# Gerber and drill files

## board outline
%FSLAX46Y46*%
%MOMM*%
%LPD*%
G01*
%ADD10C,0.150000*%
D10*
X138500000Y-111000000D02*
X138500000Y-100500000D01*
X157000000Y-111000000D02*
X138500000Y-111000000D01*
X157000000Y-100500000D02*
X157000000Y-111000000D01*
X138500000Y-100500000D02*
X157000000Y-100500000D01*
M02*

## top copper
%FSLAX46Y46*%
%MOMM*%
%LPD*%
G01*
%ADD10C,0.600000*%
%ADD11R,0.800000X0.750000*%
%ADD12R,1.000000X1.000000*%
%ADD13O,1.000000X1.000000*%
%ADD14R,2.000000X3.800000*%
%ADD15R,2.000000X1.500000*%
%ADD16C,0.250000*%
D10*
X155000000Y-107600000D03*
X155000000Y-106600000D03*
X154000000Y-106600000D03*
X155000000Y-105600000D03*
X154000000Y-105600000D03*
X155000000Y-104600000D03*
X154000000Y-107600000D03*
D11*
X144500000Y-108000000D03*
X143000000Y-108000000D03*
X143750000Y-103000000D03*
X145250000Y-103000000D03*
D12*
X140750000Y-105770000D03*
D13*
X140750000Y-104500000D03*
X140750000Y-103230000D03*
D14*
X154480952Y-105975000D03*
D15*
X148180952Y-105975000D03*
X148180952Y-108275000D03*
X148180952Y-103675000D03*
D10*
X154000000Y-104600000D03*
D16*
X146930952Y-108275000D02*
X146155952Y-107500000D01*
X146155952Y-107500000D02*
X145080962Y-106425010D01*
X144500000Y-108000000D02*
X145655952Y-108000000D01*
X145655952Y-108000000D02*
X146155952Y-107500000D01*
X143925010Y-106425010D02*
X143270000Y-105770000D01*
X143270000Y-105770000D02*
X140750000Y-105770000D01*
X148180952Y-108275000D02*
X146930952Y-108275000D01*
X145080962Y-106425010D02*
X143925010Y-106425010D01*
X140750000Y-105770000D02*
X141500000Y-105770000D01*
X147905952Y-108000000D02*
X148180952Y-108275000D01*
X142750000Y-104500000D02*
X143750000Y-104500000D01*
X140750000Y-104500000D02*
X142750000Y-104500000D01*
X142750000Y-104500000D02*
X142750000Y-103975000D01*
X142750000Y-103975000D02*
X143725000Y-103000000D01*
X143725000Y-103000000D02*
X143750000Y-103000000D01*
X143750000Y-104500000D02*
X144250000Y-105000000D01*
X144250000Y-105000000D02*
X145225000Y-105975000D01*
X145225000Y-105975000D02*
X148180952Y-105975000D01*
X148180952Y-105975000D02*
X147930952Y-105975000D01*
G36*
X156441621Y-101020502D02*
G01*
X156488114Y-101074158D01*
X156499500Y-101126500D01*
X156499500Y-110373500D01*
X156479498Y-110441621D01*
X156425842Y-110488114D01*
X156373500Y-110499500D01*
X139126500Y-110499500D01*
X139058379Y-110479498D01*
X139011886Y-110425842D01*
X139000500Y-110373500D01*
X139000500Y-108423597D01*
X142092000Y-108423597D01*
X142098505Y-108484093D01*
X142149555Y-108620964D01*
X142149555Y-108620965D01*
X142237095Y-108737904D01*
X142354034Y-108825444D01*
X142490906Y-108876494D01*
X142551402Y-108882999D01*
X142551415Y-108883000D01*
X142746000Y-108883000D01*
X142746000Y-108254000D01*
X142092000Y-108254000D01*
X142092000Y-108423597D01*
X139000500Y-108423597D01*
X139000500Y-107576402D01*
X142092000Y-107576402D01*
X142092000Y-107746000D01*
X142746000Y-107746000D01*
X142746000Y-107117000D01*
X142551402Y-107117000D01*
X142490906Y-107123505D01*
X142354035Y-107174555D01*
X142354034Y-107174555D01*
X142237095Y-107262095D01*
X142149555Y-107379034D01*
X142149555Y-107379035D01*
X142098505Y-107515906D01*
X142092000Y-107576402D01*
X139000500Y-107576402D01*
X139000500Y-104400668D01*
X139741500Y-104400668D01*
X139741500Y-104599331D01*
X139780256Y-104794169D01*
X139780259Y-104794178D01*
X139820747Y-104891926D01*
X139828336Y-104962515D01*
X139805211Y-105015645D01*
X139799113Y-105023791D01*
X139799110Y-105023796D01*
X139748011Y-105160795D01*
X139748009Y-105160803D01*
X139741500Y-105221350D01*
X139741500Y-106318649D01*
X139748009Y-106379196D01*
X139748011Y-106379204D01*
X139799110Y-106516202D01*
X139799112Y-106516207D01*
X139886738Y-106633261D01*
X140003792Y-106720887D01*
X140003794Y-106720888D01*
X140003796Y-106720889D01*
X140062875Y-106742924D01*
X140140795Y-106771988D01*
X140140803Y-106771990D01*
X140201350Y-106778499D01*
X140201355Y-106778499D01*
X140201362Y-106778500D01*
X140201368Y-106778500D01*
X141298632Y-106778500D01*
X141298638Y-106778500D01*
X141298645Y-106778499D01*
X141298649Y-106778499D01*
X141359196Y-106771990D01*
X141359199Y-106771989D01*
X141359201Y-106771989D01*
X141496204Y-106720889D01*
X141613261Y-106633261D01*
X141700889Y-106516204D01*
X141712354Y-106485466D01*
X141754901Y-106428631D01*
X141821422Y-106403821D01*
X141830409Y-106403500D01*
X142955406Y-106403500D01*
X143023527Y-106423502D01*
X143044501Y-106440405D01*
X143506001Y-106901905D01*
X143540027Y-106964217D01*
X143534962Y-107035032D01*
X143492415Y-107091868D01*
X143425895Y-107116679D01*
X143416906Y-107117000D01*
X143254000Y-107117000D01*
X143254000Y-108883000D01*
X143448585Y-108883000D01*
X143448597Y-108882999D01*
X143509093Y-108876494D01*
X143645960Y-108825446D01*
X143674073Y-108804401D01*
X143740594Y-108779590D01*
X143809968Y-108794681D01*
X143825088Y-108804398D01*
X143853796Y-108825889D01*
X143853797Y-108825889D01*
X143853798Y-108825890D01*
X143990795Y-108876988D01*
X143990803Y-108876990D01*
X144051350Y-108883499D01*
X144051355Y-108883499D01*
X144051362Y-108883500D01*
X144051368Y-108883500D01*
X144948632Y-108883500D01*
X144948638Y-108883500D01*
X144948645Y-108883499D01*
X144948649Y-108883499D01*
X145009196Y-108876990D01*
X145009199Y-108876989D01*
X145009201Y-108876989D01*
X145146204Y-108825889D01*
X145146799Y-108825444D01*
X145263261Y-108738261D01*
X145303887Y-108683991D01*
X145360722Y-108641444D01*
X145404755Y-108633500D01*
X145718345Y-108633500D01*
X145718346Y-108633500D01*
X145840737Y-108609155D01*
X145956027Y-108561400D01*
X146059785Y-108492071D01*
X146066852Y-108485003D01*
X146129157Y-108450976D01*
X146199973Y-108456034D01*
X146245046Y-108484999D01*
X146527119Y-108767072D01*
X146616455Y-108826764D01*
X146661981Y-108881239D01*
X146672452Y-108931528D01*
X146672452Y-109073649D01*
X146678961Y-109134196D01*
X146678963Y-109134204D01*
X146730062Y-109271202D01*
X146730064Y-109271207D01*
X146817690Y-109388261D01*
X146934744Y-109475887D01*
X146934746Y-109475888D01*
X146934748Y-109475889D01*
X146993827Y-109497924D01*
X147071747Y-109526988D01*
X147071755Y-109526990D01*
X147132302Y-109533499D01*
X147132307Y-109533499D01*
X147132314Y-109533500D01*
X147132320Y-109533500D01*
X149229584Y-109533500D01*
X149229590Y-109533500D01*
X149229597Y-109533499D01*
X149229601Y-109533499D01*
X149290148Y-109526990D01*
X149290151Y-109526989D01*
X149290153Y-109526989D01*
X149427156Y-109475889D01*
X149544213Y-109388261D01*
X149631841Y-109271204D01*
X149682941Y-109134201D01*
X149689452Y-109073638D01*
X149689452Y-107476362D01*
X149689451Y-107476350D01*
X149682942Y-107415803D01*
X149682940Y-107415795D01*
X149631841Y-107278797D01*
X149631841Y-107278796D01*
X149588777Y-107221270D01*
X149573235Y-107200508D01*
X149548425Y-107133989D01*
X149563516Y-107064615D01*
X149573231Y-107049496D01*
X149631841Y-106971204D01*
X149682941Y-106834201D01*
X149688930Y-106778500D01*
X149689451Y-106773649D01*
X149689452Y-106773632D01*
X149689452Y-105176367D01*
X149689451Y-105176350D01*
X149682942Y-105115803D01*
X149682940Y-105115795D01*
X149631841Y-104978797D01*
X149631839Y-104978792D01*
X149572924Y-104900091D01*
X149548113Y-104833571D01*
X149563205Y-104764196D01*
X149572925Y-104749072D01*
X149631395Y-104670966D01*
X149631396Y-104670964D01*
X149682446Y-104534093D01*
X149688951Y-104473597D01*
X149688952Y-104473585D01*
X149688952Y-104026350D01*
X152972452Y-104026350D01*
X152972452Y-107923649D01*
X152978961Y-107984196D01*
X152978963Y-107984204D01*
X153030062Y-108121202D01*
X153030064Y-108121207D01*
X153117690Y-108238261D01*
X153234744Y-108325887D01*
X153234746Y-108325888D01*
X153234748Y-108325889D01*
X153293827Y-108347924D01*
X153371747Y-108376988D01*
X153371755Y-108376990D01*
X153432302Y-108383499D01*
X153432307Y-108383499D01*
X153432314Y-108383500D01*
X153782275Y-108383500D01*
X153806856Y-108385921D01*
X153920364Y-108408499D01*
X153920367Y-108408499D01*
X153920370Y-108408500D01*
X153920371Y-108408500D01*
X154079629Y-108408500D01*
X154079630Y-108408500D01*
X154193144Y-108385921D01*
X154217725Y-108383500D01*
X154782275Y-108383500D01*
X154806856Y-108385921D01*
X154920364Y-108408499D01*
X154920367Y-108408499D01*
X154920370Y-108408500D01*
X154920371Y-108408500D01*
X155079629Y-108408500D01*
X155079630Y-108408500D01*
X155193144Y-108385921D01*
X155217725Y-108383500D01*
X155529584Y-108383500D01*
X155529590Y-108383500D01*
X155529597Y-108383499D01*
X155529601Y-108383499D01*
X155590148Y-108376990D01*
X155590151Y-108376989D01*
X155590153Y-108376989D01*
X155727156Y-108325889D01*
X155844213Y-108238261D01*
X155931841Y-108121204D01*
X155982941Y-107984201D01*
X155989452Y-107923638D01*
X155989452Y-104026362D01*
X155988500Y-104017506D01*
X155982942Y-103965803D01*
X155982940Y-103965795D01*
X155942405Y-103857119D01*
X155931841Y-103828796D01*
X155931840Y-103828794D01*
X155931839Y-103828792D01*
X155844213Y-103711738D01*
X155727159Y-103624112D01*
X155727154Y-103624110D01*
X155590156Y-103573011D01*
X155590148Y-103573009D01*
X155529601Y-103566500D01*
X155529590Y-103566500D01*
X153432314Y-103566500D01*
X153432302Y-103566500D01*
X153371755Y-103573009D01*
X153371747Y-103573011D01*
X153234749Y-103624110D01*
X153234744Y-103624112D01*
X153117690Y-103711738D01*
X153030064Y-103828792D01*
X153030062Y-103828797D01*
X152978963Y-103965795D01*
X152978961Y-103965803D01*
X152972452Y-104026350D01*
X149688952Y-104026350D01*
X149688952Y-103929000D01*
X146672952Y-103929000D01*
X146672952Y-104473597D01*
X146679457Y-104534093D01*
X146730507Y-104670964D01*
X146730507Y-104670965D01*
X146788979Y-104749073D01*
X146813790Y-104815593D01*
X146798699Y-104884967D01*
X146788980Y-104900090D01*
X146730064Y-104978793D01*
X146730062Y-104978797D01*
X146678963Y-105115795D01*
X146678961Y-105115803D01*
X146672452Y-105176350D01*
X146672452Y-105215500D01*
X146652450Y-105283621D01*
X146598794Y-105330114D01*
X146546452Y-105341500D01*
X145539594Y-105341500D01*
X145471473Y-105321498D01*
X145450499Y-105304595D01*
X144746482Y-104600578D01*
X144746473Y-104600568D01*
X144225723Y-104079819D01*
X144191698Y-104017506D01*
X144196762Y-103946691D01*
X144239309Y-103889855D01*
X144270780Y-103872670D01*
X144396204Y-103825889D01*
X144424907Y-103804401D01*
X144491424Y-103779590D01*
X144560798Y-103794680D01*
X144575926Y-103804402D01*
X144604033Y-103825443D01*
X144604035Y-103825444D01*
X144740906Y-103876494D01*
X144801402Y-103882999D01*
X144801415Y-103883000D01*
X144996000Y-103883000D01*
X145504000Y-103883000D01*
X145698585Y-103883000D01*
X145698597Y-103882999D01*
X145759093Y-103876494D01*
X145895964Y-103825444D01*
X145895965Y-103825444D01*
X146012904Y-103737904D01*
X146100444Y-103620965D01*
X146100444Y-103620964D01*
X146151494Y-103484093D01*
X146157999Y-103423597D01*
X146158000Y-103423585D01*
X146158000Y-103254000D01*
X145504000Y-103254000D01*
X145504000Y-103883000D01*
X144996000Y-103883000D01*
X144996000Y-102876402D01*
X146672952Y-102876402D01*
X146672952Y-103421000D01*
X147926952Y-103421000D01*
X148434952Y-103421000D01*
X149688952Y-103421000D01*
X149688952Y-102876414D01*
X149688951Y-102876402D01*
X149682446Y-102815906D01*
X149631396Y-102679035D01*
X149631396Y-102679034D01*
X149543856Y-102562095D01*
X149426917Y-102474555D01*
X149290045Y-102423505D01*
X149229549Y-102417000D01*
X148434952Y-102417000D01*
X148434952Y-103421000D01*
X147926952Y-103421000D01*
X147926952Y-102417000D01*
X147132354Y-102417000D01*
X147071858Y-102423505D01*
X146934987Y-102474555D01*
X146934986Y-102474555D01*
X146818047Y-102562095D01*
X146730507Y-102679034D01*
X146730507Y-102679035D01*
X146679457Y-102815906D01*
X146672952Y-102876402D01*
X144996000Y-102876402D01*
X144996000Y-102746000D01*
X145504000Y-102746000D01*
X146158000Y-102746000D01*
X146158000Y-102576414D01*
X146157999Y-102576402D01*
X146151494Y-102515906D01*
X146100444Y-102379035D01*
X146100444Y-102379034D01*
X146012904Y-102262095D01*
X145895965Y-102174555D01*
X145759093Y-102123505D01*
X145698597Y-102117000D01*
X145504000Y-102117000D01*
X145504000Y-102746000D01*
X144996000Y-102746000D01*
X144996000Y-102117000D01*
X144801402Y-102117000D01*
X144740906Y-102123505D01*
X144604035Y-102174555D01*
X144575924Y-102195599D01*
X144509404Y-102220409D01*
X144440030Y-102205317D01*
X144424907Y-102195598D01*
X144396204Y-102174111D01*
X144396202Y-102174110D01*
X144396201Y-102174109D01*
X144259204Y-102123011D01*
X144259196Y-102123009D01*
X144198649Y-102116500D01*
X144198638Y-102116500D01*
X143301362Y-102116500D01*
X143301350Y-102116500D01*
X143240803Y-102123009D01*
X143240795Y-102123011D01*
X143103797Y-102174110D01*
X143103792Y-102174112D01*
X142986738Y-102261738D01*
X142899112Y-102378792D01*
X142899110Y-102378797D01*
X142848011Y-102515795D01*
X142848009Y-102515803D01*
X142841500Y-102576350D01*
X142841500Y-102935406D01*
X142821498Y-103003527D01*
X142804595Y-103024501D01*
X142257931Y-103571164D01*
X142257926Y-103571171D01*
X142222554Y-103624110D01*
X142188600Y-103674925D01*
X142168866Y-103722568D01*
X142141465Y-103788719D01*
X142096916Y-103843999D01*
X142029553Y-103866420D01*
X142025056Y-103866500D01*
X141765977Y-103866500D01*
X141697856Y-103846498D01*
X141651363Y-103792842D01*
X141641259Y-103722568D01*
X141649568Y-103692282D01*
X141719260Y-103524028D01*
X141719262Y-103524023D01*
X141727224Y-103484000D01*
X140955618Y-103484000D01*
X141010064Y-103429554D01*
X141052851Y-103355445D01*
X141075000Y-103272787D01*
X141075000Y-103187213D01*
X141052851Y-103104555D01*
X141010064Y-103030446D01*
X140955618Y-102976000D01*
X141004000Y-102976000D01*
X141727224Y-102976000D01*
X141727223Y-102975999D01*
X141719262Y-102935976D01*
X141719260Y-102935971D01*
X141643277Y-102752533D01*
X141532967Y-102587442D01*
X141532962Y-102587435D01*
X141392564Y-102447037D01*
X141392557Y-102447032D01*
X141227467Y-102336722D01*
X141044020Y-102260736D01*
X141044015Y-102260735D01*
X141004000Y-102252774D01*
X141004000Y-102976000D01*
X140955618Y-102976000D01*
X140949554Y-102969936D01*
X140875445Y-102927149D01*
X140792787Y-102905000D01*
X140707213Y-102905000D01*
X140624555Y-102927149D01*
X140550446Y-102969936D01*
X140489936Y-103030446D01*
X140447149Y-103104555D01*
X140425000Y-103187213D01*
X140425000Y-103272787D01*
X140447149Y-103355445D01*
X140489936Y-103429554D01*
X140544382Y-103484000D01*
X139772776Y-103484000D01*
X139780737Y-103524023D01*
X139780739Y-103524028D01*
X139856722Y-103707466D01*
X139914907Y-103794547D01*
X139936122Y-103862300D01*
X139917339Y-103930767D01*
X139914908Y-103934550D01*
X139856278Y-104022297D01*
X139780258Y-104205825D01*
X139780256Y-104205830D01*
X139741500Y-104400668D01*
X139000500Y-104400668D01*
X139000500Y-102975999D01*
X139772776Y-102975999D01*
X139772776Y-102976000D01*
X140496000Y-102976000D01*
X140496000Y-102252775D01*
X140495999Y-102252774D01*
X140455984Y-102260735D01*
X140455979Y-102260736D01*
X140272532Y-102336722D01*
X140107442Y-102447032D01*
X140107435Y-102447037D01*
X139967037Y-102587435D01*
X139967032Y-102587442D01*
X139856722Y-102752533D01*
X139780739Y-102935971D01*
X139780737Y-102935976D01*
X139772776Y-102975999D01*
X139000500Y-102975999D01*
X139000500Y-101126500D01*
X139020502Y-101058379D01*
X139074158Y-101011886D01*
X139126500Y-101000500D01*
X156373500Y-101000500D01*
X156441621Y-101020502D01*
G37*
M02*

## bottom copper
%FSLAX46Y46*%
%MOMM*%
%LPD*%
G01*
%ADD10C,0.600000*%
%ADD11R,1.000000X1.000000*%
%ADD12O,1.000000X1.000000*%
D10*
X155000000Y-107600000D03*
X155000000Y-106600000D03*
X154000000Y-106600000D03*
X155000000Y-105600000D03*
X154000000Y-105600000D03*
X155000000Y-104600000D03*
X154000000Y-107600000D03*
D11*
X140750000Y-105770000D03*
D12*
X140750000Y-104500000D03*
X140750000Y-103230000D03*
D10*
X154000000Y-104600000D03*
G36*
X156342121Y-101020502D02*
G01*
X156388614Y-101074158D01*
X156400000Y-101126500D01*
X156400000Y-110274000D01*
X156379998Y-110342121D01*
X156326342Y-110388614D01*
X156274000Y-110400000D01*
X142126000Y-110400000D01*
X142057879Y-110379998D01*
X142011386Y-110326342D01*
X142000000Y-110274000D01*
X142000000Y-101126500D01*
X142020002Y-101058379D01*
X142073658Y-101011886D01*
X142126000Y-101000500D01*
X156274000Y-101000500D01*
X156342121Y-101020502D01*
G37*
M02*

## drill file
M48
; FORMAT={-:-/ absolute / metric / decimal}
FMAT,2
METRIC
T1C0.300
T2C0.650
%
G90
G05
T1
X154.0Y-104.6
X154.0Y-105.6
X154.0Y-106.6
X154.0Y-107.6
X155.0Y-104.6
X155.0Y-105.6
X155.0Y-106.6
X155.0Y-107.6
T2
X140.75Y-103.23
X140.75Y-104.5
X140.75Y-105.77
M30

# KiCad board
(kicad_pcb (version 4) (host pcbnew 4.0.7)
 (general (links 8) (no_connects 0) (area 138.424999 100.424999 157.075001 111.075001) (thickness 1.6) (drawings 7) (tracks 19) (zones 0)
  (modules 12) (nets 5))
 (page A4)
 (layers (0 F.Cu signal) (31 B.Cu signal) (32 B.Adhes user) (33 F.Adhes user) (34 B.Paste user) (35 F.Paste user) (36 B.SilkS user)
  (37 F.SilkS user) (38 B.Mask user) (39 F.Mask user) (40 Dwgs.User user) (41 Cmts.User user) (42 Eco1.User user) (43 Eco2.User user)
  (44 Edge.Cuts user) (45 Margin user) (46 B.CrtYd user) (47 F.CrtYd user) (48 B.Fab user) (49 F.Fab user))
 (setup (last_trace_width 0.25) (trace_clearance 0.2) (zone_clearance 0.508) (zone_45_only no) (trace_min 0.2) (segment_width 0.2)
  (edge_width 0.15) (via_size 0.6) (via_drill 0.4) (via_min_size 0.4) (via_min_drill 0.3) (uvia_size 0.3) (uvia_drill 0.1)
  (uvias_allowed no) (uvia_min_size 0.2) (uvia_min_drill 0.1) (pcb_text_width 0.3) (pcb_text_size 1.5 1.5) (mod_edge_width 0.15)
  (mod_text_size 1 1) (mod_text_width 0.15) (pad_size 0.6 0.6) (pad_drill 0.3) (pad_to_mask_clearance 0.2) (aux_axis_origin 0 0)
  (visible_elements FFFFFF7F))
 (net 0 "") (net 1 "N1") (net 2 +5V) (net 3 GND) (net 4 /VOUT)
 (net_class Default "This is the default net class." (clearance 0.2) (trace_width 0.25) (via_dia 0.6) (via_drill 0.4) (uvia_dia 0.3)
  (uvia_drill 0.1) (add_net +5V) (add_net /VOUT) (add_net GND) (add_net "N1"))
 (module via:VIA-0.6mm (layer F.Cu) (at 155 107.6)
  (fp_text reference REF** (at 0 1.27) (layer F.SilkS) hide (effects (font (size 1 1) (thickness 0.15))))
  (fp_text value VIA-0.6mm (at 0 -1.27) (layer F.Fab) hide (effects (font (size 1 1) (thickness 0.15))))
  (pad 1 thru_hole circle (at 0 0) (size 0.6 0.6) (drill 0.3) (layers *.Cu) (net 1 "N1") (zone_connect 2)))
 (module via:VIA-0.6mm (layer F.Cu) (at 155 106.6)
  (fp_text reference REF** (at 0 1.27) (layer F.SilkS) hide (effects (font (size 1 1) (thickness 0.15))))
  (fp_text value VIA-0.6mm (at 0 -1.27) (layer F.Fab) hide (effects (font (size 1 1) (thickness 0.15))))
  (pad 1 thru_hole circle (at 0 0) (size 0.6 0.6) (drill 0.3) (layers *.Cu) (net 1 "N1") (zone_connect 2)))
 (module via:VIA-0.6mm (layer F.Cu) (at 154 106.6)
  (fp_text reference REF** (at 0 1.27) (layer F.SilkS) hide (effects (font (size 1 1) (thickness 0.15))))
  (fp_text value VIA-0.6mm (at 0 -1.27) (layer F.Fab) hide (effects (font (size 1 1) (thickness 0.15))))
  (pad 1 thru_hole circle (at 0 0) (size 0.6 0.6) (drill 0.3) (layers *.Cu) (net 1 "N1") (zone_connect 2)))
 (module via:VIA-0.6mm (layer F.Cu) (at 155 105.6)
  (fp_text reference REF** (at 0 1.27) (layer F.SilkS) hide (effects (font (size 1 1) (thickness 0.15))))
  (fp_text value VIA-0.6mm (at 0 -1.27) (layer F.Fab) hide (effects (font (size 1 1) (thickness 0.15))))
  (pad 1 thru_hole circle (at 0 0) (size 0.6 0.6) (drill 0.3) (layers *.Cu) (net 1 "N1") (zone_connect 2)))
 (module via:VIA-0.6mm (layer F.Cu) (at 154 105.6)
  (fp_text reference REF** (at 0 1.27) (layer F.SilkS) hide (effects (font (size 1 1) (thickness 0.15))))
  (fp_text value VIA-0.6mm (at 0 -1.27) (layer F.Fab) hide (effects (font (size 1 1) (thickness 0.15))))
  (pad 1 thru_hole circle (at 0 0) (size 0.6 0.6) (drill 0.3) (layers *.Cu) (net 1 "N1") (zone_connect 2)))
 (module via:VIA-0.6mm (layer F.Cu) (at 155 104.6)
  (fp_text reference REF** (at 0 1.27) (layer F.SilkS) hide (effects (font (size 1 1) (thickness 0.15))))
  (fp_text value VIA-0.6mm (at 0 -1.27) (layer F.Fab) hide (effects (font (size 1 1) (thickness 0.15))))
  (pad 1 thru_hole circle (at 0 0) (size 0.6 0.6) (drill 0.3) (layers *.Cu) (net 1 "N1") (zone_connect 2)))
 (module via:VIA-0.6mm (layer F.Cu) (at 154 107.6)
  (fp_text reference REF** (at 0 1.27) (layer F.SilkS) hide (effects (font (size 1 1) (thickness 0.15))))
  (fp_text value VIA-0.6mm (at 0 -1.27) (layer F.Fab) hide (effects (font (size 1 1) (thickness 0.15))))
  (pad 1 thru_hole circle (at 0 0) (size 0.6 0.6) (drill 0.3) (layers *.Cu) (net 1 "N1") (zone_connect 2)))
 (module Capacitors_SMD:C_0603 (layer F.Cu) (at 143.75 108 180)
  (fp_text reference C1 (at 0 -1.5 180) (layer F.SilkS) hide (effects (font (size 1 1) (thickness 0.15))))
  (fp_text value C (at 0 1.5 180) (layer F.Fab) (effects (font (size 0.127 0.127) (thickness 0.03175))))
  (pad 1 smd rect (at -0.75 0 180) (size 0.8 0.75) (layers F.Cu F.Paste F.Mask) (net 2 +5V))
  (pad 2 smd rect (at 0.75 0 180) (size 0.8 0.75) (layers F.Cu F.Paste F.Mask) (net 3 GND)))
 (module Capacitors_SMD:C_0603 (layer F.Cu) (at 144.5 103)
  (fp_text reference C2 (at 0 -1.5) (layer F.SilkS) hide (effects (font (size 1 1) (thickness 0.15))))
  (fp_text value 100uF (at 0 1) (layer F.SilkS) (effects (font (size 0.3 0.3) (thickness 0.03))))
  (pad 1 smd rect (at -0.75 0) (size 0.8 0.75) (layers F.Cu F.Paste F.Mask) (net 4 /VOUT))
  (pad 2 smd rect (at 0.75 0) (size 0.8 0.75) (layers F.Cu F.Paste F.Mask) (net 3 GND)))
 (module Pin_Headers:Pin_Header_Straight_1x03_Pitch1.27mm (layer F.Cu) (at 140.75 105.77 180)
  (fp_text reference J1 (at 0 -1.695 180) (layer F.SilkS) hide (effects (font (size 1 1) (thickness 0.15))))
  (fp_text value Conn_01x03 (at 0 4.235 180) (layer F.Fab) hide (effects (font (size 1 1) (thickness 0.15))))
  (pad 1 thru_hole rect (at 0 0 180) (size 1 1) (drill 0.65) (layers *.Cu *.Mask) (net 2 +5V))
  (pad 2 thru_hole oval (at 0 1.27 180) (size 1 1) (drill 0.65) (layers *.Cu *.Mask) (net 4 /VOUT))
  (pad 3 thru_hole oval (at 0 2.54 180) (size 1 1) (drill 0.65) (layers *.Cu *.Mask) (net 3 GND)))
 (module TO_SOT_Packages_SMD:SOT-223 (layer F.Cu) (at 151.330952 105.975)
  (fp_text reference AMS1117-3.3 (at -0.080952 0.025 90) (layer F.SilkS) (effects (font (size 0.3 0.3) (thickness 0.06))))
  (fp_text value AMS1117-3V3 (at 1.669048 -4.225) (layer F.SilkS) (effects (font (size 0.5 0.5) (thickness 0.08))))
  (pad 4 smd rect (at 3.15 0) (size 2 3.8) (layers F.Cu F.Paste F.Mask) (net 1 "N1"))
  (pad 2 smd rect (at -3.15 0) (size 2 1.5) (layers F.Cu F.Paste F.Mask) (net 4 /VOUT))
  (pad 3 smd rect (at -3.15 2.3) (size 2 1.5) (layers F.Cu F.Paste F.Mask) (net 2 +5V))
  (pad 1 smd rect (at -3.15 -2.3) (size 2 1.5) (layers F.Cu F.Paste F.Mask) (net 3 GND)))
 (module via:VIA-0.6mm (layer F.Cu) (at 154 104.6)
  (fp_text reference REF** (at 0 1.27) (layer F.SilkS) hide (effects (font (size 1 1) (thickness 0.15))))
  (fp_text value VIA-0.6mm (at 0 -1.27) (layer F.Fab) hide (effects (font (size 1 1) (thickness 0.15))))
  (pad 1 thru_hole circle (at 0 0) (size 0.6 0.6) (drill 0.3) (layers *.Cu) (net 1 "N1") (zone_connect 2)))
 (gr_line (start 138.5 111) (end 138.5 100.5) (angle 90) (layer Edge.Cuts) (width 0.15))
 (gr_line (start 157 111) (end 138.5 111) (angle 90) (layer Edge.Cuts) (width 0.15))
 (gr_line (start 157 100.5) (end 157 111) (angle 90) (layer Edge.Cuts) (width 0.15))
 (gr_line (start 138.5 100.5) (end 157 100.5) (angle 90) (layer Edge.Cuts) (width 0.15))
 (segment (start 146.930952 108.275) (end 146.155952 107.5) (width 0.25) (layer F.Cu) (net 2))
 (segment (start 146.155952 107.5) (end 145.080962 106.42501) (width 0.25) (layer F.Cu) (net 2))
 (segment (start 144.5 108) (end 145.655952 108) (width 0.25) (layer F.Cu) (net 2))
 (segment (start 145.655952 108) (end 146.155952 107.5) (width 0.25) (layer F.Cu) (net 2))
 (segment (start 143.92501 106.42501) (end 143.27 105.77) (width 0.25) (layer F.Cu) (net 2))
 (segment (start 143.27 105.77) (end 140.75 105.77) (width 0.25) (layer F.Cu) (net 2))
 (segment (start 148.180952 108.275) (end 146.930952 108.275) (width 0.25) (layer F.Cu) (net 2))
 (segment (start 145.080962 106.42501) (end 143.92501 106.42501) (width 0.25) (layer F.Cu) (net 2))
 (segment (start 140.75 105.77) (end 141.5 105.77) (width 0.25) (layer F.Cu) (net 2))
 (segment (start 147.905952 108) (end 148.180952 108.275) (width 0.25) (layer F.Cu) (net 2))
 (segment (start 142.75 104.5) (end 143.75 104.5) (width 0.25) (layer F.Cu) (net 4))
 (segment (start 140.75 104.5) (end 142.75 104.5) (width 0.25) (layer F.Cu) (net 4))
 (segment (start 142.75 104.5) (end 142.75 103.975) (width 0.25) (layer F.Cu) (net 4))
 (segment (start 142.75 103.975) (end 143.725 103) (width 0.25) (layer F.Cu) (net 4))
 (segment (start 143.725 103) (end 143.75 103) (width 0.25) (layer F.Cu) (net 4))
 (segment (start 143.75 104.5) (end 144.25 105) (width 0.25) (layer F.Cu) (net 4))
 (segment (start 144.25 105) (end 145.225 105.975) (width 0.25) (layer F.Cu) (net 4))
 (segment (start 145.225 105.975) (end 148.180952 105.975) (width 0.25) (layer F.Cu) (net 4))
 (segment (start 148.180952 105.975) (end 147.930952 105.975) (width 0.25) (layer F.Cu) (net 4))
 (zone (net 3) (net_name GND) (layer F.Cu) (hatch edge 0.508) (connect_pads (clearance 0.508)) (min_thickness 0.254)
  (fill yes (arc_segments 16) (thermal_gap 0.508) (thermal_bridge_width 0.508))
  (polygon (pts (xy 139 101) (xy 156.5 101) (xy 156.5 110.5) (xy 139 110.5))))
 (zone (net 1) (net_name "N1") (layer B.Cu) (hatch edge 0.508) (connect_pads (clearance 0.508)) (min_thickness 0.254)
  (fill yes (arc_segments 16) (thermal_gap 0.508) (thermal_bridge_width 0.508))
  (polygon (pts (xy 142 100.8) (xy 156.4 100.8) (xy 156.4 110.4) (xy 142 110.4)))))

